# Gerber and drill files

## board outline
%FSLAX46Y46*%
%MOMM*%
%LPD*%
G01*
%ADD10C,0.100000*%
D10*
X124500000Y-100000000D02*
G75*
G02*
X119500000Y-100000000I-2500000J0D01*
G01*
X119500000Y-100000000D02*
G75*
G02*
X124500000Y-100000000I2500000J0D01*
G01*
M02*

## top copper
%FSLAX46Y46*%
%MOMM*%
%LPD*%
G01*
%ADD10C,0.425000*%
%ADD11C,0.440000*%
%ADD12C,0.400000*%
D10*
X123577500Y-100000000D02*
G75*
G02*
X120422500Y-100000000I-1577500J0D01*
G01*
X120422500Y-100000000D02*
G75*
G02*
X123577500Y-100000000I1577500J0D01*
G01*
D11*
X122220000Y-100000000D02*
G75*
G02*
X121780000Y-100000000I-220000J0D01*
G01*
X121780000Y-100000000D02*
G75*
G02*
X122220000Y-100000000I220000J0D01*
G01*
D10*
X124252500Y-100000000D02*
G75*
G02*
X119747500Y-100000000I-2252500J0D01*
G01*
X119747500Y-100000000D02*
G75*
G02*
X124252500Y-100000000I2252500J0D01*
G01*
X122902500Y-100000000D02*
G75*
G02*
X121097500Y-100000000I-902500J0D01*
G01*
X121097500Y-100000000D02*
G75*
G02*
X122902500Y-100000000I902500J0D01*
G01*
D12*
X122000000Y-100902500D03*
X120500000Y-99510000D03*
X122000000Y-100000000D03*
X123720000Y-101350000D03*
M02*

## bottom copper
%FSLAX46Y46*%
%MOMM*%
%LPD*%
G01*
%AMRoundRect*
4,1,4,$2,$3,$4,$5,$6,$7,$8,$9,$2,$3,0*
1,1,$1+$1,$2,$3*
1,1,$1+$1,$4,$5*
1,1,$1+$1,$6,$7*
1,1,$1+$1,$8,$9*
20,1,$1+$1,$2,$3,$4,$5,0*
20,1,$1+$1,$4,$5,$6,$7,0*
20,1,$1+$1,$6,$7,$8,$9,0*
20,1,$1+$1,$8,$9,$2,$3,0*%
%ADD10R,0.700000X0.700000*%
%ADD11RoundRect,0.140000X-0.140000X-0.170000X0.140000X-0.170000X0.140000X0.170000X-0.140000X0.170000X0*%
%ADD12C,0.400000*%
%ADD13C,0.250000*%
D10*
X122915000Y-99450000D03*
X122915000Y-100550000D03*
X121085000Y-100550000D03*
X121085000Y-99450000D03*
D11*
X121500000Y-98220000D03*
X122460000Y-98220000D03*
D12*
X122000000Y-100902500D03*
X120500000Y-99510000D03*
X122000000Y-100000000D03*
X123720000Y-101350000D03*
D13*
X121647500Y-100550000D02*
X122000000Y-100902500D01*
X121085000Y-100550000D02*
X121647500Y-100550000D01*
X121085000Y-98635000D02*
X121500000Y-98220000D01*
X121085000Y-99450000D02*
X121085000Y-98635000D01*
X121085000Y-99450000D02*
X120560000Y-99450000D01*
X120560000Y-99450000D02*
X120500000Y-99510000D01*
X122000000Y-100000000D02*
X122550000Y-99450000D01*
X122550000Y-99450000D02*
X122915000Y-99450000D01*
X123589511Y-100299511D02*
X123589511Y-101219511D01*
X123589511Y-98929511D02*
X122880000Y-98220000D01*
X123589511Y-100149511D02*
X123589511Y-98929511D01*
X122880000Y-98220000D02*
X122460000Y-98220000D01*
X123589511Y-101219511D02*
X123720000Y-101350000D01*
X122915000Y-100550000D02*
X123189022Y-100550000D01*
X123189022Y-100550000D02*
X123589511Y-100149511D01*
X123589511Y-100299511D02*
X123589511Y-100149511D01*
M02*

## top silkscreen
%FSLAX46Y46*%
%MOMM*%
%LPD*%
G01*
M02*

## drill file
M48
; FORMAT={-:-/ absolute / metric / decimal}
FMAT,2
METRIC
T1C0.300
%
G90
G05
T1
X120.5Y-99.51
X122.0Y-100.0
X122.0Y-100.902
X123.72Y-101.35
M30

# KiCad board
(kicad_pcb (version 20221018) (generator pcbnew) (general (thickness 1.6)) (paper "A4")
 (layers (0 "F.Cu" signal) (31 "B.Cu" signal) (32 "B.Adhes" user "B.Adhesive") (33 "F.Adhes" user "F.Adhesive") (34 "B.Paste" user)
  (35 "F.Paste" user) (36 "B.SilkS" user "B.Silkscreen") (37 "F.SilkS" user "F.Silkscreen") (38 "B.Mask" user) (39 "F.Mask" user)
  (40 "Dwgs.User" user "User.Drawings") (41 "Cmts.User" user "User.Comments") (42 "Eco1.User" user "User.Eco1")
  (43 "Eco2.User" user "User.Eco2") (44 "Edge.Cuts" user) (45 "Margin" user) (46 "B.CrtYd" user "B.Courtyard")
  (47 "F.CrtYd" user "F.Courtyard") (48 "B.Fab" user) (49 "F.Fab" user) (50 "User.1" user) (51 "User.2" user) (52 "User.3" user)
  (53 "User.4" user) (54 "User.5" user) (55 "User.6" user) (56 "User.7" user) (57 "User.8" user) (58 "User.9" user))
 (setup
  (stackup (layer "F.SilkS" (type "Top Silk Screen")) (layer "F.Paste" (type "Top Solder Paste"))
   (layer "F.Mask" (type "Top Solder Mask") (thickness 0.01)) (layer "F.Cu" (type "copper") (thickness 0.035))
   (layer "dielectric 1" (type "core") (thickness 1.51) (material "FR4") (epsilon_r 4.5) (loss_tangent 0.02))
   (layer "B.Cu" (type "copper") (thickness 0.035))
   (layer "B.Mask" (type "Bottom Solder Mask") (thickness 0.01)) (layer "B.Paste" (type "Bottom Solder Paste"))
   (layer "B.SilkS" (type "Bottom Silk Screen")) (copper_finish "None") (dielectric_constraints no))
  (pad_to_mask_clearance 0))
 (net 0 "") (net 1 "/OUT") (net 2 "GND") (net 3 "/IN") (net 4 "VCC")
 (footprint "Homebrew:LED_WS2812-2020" (layer "B.Cu") (at 122 100 180)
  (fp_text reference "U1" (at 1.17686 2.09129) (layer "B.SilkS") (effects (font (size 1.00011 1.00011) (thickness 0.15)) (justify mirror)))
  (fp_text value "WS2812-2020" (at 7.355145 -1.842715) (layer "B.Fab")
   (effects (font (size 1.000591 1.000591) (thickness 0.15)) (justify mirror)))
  (pad "1" smd rect (at -0.915 0.55 180) (size 0.7 0.7) (layers "B.Cu" "B.Paste" "B.Mask") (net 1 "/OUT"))
  (pad "2" smd rect (at -0.915 -0.55 180) (size 0.7 0.7) (layers "B.Cu" "B.Paste" "B.Mask") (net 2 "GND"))
  (pad "3" smd rect (at 0.915 -0.55) (size 0.7 0.7) (layers "B.Cu" "B.Paste" "B.Mask") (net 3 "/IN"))
  (pad "4" smd rect (at 0.915 0.55) (size 0.7 0.7) (layers "B.Cu" "B.Paste" "B.Mask") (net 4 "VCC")))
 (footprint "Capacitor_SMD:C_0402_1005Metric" (layer "B.Cu") (at 121.98 98.22)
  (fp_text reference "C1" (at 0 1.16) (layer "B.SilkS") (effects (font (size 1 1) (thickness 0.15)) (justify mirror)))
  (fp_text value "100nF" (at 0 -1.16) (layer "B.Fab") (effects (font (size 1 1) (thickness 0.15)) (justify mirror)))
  (pad "1" smd roundrect (at -0.48 0) (size 0.56 0.62) (layers "B.Cu" "B.Paste" "B.Mask") (roundrect_rratio 0.25) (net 4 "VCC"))
  (pad "2" smd roundrect (at 0.48 0) (size 0.56 0.62) (layers "B.Cu" "B.Paste" "B.Mask") (roundrect_rratio 0.25) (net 2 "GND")))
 (gr_circle (center 122 100) (end 123.5775 100) (stroke (width 0.425) (type solid)) (fill none) (layer "F.Cu"))
 (gr_circle (center 122 100) (end 122.39 100) (stroke (width 0.1) (type solid)) (fill solid) (layer "F.Cu"))
 (gr_circle (center 122 100) (end 124.2525 100) (stroke (width 0.425) (type solid)) (fill none) (layer "F.Cu"))
 (gr_circle (center 122 100) (end 122.9025 100) (stroke (width 0.425) (type solid)) (fill none) (layer "F.Cu"))
 (gr_circle (center 122 100) (end 124.5 100) (stroke (width 0.1) (type solid)) (fill none) (layer "Edge.Cuts"))
 (via (at 122 100.9025) (size 0.4) (drill 0.3) (layers "F.Cu" "B.Cu") (free) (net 3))
 (segment (start 121.6475 100.55) (end 122 100.9025) (width 0.25) (layer "B.Cu") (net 3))
 (segment (start 121.085 100.55) (end 121.6475 100.55) (width 0.25) (layer "B.Cu") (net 3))
 (via (at 120.5 99.51) (size 0.4) (drill 0.3) (layers "F.Cu" "B.Cu") (free) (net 4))
 (segment (start 121.085 98.635) (end 121.5 98.22) (width 0.25) (layer "B.Cu") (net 4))
 (segment (start 121.085 99.45) (end 121.085 98.635) (width 0.25) (layer "B.Cu") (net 4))
 (segment (start 121.085 99.45) (end 120.56 99.45) (width 0.25) (layer "B.Cu") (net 4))
 (segment (start 120.56 99.45) (end 120.5 99.51) (width 0.25) (layer "B.Cu") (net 4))
 (via (at 122 100) (size 0.4) (drill 0.3) (layers "F.Cu" "B.Cu") (free) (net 1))
 (segment (start 122 100) (end 122.55 99.45) (width 0.25) (layer "B.Cu") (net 1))
 (segment (start 122.55 99.45) (end 122.915 99.45) (width 0.25) (layer "B.Cu") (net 1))
 (via (at 123.72 101.35) (size 0.4) (drill 0.3) (layers "F.Cu" "B.Cu") (free) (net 2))
 (segment (start 123.589511 100.299511) (end 123.589511 101.219511) (width 0.25) (layer "B.Cu") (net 2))
 (segment (start 123.589511 98.929511) (end 122.88 98.22) (width 0.25) (layer "B.Cu") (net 2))
 (segment (start 123.589511 100.149511) (end 123.589511 98.929511) (width 0.25) (layer "B.Cu") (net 2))
 (segment (start 122.88 98.22) (end 122.46 98.22) (width 0.25) (layer "B.Cu") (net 2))
 (segment (start 123.589511 101.219511) (end 123.72 101.35) (width 0.25) (layer "B.Cu") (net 2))
 (segment (start 122.915 100.55) (end 123.189022 100.55) (width 0.25) (layer "B.Cu") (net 2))
 (segment (start 123.189022 100.55) (end 123.589511 100.149511) (width 0.25) (layer "B.Cu") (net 2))
 (segment (start 123.589511 100.299511) (end 123.589511 100.149511) (width 0.25) (layer "B.Cu") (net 2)))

